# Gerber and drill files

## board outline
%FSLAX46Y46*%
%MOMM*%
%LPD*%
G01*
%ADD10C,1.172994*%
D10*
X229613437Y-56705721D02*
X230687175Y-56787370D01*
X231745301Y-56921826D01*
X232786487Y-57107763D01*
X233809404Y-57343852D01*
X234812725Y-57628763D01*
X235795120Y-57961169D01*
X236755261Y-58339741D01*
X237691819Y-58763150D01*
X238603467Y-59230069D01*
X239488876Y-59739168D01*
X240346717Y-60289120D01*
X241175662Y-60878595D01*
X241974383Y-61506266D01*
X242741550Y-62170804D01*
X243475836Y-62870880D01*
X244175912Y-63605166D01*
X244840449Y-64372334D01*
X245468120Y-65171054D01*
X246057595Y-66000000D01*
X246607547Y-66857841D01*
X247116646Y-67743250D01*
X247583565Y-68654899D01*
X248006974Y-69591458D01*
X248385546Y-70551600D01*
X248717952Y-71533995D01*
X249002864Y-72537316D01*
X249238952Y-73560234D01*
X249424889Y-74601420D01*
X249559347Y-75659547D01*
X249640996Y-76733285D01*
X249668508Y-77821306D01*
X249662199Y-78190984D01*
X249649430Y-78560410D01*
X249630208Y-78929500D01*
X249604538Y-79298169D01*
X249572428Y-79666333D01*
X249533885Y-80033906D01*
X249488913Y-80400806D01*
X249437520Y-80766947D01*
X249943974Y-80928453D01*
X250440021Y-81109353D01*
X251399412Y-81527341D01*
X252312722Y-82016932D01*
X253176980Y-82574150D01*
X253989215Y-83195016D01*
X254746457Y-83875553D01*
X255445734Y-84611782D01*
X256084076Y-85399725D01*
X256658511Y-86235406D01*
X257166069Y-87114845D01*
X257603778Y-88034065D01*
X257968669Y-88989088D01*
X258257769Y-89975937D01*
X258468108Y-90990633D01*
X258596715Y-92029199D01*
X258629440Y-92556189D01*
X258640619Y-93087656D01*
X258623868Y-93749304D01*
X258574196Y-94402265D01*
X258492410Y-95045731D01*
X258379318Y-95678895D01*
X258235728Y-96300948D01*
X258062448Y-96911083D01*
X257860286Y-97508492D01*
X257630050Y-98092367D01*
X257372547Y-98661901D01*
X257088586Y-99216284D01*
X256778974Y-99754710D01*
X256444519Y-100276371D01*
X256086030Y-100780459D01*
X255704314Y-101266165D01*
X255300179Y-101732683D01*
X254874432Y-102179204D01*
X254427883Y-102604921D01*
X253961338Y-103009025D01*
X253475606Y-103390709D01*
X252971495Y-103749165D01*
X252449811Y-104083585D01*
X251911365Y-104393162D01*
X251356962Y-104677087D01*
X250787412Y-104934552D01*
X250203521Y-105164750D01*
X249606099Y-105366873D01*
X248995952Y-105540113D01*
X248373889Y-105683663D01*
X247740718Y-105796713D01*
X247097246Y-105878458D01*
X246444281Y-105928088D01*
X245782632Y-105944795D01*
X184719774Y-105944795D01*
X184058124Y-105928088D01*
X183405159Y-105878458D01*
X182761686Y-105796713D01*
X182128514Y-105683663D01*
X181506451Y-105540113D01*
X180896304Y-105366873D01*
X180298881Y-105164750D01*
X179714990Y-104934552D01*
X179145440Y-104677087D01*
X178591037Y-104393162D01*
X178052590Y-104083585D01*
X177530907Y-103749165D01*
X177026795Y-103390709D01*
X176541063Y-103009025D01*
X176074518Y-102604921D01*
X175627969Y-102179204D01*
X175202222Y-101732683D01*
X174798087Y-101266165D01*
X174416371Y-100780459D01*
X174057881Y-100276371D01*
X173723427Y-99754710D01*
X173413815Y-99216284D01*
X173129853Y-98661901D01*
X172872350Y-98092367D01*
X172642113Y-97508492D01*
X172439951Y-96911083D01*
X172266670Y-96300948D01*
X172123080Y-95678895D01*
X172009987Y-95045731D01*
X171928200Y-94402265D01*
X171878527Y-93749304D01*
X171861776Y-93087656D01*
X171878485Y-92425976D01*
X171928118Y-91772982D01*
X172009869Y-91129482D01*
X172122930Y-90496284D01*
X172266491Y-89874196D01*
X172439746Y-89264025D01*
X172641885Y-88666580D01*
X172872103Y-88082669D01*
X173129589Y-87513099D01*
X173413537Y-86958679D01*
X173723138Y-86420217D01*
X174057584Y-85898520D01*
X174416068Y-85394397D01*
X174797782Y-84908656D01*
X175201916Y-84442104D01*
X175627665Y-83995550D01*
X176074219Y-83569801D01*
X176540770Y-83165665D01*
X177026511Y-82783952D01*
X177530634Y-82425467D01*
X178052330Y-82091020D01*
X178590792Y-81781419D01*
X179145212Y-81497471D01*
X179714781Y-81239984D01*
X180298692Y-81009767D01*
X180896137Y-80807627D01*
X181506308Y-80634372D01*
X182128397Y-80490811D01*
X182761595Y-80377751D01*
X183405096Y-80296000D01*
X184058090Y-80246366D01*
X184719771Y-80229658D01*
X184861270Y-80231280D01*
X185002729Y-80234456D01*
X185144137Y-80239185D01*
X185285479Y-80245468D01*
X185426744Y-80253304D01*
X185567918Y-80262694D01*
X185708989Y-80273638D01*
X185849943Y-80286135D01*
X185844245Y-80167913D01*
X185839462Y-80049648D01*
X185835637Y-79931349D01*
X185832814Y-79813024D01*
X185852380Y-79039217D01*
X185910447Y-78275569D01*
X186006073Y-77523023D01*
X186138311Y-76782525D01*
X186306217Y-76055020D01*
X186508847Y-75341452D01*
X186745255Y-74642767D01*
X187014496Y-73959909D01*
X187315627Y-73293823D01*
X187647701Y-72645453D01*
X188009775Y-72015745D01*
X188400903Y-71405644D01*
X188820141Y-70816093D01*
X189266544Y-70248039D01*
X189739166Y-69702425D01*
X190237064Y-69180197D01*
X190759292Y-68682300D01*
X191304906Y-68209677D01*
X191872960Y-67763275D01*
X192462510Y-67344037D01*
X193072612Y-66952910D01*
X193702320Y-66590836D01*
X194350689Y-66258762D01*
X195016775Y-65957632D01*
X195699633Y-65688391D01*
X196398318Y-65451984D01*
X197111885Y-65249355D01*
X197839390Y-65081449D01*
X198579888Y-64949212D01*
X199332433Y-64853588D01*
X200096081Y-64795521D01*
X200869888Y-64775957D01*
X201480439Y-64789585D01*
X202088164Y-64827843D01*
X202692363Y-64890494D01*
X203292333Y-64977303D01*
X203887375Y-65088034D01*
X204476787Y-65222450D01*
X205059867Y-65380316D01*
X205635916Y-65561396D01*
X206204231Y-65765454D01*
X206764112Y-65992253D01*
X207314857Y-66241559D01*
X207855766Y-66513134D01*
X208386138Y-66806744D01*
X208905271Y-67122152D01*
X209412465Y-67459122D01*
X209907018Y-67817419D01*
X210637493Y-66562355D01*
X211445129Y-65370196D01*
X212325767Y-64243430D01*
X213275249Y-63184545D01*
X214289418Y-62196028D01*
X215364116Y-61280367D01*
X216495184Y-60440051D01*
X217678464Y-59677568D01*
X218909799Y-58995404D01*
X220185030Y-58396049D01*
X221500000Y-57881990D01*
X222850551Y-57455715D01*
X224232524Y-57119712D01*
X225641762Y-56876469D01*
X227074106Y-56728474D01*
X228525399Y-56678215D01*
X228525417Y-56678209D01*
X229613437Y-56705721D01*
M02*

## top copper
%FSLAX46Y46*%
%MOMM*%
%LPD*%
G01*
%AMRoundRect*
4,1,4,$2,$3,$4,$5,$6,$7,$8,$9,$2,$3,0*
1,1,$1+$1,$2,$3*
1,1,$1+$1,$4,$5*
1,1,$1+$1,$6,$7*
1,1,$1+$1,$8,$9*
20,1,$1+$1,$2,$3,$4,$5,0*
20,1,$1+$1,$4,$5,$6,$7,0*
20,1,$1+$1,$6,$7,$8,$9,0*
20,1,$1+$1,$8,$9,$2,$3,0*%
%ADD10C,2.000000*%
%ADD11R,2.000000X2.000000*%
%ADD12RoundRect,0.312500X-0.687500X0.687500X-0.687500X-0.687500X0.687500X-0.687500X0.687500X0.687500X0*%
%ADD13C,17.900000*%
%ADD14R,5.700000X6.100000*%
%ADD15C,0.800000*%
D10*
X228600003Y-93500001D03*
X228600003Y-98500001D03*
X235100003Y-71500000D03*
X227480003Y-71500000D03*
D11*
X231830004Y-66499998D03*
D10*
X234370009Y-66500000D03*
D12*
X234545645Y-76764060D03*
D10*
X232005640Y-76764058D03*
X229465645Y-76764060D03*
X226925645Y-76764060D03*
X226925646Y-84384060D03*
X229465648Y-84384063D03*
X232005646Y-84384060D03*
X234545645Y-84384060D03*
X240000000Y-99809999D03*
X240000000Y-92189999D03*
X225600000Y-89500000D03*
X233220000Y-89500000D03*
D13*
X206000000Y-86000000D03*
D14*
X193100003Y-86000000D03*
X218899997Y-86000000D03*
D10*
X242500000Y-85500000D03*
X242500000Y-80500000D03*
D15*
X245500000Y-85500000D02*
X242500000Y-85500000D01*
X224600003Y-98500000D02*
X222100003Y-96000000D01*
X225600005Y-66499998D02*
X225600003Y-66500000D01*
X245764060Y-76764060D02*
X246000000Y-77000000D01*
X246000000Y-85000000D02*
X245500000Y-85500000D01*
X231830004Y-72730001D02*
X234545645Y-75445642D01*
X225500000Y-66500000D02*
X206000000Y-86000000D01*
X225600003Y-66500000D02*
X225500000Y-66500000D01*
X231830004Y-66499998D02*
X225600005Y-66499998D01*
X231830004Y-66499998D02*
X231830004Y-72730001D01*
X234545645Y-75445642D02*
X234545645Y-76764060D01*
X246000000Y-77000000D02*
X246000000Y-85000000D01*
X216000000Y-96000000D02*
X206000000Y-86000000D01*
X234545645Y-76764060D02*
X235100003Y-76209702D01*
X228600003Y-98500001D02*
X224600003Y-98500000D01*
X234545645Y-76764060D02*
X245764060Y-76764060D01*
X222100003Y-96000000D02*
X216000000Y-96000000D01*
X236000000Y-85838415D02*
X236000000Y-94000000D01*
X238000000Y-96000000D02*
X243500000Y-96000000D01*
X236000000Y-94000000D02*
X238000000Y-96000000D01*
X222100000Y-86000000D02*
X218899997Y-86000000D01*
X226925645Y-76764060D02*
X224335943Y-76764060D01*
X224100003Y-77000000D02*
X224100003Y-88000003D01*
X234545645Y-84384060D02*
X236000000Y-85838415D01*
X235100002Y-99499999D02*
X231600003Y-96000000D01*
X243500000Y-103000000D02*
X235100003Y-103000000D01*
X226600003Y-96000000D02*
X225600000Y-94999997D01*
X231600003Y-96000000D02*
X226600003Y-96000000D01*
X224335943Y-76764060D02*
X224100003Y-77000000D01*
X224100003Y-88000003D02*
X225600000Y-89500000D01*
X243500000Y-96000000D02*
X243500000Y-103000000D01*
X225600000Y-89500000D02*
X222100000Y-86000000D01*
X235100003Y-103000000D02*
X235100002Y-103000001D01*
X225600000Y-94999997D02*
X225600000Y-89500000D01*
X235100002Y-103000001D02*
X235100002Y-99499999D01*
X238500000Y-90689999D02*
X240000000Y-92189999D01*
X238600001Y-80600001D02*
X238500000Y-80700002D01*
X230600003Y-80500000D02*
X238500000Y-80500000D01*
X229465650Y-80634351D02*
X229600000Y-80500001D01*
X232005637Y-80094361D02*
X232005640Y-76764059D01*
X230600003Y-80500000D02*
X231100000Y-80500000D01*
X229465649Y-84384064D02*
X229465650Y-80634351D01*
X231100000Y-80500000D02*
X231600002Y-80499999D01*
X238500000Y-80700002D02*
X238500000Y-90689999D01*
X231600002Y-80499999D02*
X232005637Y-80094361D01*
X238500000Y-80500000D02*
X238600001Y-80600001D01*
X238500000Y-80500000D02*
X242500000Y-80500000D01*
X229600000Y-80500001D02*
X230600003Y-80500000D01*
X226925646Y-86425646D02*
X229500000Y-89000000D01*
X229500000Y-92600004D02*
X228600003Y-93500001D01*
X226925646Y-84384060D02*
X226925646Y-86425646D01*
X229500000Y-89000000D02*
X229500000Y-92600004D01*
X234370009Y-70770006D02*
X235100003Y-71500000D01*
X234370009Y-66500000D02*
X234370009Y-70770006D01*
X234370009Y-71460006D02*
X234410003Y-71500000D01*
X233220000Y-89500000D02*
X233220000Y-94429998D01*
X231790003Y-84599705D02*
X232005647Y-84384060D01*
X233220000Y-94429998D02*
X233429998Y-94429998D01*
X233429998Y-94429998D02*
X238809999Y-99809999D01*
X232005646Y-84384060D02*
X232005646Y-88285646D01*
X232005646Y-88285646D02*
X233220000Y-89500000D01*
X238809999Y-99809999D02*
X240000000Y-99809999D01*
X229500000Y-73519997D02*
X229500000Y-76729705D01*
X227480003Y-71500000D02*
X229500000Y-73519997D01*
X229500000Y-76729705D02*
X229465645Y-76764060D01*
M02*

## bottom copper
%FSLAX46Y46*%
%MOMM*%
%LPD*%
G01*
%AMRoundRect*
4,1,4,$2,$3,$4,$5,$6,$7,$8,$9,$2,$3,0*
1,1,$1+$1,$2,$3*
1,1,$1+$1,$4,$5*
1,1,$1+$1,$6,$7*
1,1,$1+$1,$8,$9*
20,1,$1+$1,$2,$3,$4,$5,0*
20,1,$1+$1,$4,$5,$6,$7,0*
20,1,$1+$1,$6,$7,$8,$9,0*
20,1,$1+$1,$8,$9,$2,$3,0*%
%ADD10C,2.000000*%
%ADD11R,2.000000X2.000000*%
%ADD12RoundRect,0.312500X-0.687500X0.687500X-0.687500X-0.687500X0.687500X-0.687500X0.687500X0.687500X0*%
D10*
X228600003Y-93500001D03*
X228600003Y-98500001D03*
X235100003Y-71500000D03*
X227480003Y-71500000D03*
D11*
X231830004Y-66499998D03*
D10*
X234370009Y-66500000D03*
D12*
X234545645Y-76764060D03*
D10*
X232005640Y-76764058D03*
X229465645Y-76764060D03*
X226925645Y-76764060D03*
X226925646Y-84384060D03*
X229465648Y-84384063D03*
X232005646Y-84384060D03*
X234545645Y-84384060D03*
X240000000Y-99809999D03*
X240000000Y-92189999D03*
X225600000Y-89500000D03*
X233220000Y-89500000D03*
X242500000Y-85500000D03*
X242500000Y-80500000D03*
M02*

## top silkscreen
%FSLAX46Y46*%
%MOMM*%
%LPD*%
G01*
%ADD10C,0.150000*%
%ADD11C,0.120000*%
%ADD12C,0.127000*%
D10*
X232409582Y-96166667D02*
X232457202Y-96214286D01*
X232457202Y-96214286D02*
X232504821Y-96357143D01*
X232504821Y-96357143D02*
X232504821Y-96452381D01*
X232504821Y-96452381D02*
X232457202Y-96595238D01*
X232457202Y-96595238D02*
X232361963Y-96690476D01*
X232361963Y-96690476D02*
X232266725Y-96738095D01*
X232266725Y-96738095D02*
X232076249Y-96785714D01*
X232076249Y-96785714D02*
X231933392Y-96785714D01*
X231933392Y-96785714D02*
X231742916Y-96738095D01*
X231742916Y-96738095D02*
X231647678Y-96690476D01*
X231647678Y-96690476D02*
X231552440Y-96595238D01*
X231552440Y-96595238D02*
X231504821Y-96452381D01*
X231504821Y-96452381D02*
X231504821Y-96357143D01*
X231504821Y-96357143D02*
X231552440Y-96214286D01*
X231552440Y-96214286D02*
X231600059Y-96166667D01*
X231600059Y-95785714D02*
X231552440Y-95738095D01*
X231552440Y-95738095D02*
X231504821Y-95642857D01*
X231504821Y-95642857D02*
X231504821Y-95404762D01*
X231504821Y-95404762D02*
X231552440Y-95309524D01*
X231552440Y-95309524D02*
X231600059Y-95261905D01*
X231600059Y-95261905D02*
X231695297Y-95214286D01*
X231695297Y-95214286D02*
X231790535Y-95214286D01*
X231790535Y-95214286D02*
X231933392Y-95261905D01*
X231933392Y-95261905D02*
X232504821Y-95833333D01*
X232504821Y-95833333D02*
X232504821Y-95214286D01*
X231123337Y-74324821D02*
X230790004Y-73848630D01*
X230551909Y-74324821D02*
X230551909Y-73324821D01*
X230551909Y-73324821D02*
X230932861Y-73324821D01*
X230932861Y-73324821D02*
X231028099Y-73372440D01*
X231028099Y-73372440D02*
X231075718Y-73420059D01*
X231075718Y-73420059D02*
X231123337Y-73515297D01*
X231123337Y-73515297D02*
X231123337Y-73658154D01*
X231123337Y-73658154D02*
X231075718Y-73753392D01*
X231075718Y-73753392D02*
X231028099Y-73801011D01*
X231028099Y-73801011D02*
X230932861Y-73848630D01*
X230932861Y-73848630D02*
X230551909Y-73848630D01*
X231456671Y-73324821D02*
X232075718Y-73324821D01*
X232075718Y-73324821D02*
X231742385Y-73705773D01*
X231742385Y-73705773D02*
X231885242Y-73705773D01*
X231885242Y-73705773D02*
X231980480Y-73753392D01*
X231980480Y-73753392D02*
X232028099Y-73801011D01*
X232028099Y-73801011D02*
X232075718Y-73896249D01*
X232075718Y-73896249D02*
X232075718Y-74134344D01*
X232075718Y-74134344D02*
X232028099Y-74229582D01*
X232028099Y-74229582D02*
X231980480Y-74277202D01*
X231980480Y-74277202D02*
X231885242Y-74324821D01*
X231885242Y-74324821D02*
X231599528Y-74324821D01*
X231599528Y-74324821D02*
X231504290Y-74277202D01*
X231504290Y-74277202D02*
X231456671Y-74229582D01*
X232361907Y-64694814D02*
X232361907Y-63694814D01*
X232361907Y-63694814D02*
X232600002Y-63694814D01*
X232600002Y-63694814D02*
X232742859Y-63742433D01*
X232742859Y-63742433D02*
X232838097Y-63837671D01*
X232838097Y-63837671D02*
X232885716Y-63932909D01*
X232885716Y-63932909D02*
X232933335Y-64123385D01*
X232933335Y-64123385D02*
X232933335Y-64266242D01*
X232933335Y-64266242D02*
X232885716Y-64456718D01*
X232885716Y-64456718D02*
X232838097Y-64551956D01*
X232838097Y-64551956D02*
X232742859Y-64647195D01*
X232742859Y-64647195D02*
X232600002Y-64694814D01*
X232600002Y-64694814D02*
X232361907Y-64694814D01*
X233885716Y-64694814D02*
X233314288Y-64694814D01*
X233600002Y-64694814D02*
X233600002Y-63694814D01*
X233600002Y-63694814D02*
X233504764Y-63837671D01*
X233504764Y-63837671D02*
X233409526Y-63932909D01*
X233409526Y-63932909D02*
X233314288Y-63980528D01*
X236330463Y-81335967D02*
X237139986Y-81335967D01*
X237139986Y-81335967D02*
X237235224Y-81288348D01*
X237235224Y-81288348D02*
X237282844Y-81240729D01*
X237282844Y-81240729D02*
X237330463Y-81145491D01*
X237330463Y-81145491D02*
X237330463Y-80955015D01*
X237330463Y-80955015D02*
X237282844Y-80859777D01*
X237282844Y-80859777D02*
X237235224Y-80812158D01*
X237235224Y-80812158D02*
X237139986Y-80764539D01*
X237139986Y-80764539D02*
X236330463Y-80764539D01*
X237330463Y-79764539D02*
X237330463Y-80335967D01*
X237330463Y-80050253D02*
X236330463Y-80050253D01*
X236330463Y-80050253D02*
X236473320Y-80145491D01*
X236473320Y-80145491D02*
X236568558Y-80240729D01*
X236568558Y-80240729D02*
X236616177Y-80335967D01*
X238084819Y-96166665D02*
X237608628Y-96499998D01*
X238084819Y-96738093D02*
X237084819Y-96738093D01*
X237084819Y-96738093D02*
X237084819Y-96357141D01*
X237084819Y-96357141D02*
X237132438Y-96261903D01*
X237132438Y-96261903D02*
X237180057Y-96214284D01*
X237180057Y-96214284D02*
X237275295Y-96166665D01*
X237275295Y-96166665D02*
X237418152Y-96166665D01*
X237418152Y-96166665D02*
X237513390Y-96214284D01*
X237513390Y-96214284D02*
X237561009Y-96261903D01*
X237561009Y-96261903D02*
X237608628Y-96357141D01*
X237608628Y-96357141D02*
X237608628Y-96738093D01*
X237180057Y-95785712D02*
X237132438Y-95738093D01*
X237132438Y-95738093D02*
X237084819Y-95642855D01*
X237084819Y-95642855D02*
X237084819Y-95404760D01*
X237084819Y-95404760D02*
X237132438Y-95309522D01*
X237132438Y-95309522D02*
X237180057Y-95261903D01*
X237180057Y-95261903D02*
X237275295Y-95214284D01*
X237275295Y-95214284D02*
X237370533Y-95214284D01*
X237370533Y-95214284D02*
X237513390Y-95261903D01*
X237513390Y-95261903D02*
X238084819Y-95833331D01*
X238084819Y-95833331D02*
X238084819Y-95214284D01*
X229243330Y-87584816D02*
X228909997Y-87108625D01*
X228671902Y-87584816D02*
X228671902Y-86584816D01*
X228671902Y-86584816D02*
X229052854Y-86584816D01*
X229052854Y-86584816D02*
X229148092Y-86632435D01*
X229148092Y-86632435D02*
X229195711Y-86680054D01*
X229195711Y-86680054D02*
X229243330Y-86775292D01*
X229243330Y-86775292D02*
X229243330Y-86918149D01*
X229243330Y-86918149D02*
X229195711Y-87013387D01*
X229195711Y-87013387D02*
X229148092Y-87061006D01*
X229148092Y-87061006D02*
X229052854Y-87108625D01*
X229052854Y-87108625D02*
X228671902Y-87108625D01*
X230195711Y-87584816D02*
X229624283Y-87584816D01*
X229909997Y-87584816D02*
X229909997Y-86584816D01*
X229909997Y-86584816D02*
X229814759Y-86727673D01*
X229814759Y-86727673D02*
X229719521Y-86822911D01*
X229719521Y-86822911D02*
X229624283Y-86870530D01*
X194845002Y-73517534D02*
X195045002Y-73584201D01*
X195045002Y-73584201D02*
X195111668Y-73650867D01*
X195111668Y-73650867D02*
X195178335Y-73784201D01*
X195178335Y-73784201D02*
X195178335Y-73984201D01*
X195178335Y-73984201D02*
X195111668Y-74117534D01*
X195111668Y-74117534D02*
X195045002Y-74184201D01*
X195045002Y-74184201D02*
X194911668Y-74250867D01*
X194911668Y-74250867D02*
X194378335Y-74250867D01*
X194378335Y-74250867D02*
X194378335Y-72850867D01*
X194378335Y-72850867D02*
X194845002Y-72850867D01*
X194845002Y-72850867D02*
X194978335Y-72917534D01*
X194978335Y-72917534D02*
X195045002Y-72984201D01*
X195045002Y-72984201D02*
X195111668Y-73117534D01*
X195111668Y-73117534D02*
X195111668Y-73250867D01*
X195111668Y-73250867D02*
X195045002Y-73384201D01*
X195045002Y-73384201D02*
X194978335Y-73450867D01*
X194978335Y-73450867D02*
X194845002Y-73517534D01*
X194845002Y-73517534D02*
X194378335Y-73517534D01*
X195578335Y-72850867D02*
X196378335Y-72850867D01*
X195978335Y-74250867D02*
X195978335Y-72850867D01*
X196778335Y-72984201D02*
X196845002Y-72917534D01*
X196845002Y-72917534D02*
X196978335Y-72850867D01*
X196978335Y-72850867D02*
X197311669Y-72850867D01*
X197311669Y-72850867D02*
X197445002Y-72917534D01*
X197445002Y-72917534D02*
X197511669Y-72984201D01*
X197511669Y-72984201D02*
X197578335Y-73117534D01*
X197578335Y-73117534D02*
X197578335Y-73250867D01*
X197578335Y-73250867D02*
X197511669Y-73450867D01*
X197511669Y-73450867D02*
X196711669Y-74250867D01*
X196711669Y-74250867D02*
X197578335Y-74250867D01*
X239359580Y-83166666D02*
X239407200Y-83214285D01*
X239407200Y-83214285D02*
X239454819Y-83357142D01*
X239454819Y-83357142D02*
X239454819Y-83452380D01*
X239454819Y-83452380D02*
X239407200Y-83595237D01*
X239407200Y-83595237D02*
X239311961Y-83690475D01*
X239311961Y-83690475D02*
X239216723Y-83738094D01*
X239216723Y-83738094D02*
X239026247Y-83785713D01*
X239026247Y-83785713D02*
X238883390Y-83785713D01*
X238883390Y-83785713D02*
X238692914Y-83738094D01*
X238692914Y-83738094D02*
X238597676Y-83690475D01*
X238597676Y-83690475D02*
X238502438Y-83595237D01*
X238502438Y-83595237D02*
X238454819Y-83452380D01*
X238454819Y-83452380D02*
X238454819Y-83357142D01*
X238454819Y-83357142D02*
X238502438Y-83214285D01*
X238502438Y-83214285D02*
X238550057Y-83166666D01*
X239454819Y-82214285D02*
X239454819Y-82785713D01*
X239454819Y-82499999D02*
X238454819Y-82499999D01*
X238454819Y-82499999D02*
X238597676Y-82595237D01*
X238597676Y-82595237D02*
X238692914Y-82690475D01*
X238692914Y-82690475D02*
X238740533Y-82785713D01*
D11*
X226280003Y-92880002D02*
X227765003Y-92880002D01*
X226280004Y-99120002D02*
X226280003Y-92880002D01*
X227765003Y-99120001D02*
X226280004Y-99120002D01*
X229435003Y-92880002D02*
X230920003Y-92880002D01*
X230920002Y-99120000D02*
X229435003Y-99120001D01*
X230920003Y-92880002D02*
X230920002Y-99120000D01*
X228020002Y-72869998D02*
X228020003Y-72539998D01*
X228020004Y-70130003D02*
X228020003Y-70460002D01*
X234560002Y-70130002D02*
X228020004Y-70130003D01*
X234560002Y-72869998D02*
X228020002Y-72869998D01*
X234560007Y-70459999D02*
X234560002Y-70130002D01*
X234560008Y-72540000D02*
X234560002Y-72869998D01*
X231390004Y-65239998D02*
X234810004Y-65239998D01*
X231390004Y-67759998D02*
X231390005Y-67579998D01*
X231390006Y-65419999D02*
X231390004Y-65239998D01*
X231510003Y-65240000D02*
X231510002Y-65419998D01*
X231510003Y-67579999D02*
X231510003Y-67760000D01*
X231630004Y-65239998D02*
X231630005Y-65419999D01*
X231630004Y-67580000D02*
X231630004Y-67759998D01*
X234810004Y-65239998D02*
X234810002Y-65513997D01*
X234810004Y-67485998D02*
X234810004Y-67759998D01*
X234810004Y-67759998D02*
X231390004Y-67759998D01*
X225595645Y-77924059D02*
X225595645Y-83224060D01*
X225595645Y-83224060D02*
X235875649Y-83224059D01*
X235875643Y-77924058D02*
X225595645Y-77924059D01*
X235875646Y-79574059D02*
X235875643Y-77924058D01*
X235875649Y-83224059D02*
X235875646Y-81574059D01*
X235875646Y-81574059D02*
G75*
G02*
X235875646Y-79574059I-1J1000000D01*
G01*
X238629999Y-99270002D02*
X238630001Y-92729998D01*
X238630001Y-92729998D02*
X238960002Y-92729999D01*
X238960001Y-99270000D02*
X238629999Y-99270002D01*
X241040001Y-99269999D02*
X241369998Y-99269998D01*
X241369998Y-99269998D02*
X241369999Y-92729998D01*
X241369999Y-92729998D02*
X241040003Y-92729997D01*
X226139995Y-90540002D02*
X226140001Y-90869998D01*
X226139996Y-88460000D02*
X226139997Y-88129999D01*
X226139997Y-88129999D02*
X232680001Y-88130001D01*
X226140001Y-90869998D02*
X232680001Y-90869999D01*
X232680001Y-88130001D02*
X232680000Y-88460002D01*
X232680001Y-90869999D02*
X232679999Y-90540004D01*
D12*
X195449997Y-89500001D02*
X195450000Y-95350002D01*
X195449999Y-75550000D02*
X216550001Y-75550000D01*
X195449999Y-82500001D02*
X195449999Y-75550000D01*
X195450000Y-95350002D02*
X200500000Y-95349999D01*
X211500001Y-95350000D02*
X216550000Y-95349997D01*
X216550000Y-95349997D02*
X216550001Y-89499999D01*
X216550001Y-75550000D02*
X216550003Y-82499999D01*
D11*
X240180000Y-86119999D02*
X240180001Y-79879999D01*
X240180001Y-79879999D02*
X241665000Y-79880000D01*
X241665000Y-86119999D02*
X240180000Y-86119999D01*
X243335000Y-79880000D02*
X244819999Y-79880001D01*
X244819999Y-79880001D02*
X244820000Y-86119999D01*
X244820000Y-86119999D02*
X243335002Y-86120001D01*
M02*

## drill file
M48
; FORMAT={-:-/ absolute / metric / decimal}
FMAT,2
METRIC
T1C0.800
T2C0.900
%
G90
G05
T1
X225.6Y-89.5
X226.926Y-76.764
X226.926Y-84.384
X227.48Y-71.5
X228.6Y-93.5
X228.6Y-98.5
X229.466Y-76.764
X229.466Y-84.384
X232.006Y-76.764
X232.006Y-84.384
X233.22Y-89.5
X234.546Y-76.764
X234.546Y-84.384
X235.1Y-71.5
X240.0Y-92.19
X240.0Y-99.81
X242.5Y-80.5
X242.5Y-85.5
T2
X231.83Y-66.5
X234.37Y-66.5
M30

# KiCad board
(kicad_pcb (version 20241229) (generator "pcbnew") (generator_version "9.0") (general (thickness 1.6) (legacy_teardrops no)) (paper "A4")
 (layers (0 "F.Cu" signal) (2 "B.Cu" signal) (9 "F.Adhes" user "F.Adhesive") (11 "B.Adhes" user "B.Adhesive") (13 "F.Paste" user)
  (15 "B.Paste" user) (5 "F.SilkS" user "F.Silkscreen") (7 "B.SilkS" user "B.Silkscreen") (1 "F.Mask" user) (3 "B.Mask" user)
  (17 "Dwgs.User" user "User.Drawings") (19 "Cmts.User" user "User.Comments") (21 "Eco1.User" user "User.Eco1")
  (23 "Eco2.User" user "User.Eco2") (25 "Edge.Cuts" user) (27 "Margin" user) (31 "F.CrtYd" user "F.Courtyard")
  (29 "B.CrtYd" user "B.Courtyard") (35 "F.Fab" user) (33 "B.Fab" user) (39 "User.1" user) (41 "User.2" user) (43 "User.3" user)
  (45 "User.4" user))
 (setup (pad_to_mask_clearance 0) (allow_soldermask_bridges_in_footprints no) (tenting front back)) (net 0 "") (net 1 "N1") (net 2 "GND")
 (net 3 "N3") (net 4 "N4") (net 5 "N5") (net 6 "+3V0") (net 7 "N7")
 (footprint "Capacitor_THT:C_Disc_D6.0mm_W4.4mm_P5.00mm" (layer "F.Cu") (at 228.600003 93.500001 -90)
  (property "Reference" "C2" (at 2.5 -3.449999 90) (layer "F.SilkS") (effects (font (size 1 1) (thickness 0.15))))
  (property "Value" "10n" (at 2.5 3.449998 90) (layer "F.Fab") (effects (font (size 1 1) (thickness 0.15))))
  (fp_line (start -0.619999 2.32) (end -0.619999 0.835) (stroke (width 0.12) (type solid)) (layer "F.SilkS"))
  (fp_line (start 5.620001 2.319999) (end -0.619999 2.32) (stroke (width 0.12) (type solid)) (layer "F.SilkS"))
  (fp_line (start 5.62 0.835) (end 5.620001 2.319999) (stroke (width 0.12) (type solid)) (layer "F.SilkS"))
  (fp_line (start -0.619999 -0.835) (end -0.619999 -2.32) (stroke (width 0.12) (type solid)) (layer "F.SilkS"))
  (fp_line (start 5.619999 -2.319999) (end 5.62 -0.835) (stroke (width 0.12) (type solid)) (layer "F.SilkS"))
  (fp_line (start -0.619999 -2.32) (end 5.619999 -2.319999) (stroke (width 0.12) (type solid)) (layer "F.SilkS"))
  (pad "1" thru_hole circle (at 0 0 270) (size 2 2) (drill 0.8) (layers "*.Cu" "*.Mask") (remove_unused_layers no) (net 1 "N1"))
  (pad "2" thru_hole circle (at 5 0 270) (size 2 2) (drill 0.8) (layers "*.Cu" "*.Mask") (remove_unused_layers no) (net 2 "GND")))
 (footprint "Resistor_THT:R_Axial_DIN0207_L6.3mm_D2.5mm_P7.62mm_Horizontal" (layer "F.Cu") (at 235.100003 71.5 180)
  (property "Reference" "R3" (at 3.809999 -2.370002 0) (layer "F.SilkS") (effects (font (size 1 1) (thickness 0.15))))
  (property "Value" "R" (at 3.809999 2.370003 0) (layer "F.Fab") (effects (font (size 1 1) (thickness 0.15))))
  (fp_line (start 7.080001 -1.369998) (end 7.08 -1.039998) (stroke (width 0.12) (type solid)) (layer "F.SilkS"))
  (fp_line (start 7.079999 1.369997) (end 7.08 1.039998) (stroke (width 0.12) (type solid)) (layer "F.SilkS"))
  (fp_line (start 0.540001 1.369998) (end 7.079999 1.369997) (stroke (width 0.12) (type solid)) (layer "F.SilkS"))
  (fp_line (start 0.540001 -1.369998) (end 7.080001 -1.369998) (stroke (width 0.12) (type solid)) (layer "F.SilkS"))
  (fp_line (start 0.539996 1.040001) (end 0.540001 1.369998) (stroke (width 0.12) (type solid)) (layer "F.SilkS"))
  (fp_line (start 0.539995 -1.04) (end 0.540001 -1.369998) (stroke (width 0.12) (type solid)) (layer "F.SilkS"))
  (pad "1" thru_hole circle (at 0 0 180) (size 2 2) (drill 0.8) (layers "*.Cu" "*.Mask") (remove_unused_layers no) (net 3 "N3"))
  (pad "2" thru_hole circle (at 7.62 0 180) (size 2 2) (drill 0.8) (layers "*.Cu" "*.Mask") (remove_unused_layers no) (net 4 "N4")))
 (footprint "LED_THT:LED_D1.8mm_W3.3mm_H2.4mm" (layer "F.Cu") (at 231.830004 66.499998)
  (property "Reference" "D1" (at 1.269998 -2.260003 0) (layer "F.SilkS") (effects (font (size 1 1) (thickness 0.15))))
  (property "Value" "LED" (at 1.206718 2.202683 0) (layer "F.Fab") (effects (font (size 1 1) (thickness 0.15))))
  (fp_line (start -0.44 -1.26) (end 2.98 -1.26) (stroke (width 0.12) (type solid)) (layer "F.SilkS"))
  (fp_line (start -0.44 1.26) (end -0.439999 1.08) (stroke (width 0.12) (type solid)) (layer "F.SilkS"))
  (fp_line (start -0.439998 -1.079999) (end -0.44 -1.26) (stroke (width 0.12) (type solid)) (layer "F.SilkS"))
  (fp_line (start -0.320001 -1.259998) (end -0.320002 -1.08) (stroke (width 0.12) (type solid)) (layer "F.SilkS"))
  (fp_line (start -0.320001 1.080001) (end -0.320001 1.260002) (stroke (width 0.12) (type solid)) (layer "F.SilkS"))
  (fp_line (start -0.2 -1.26) (end -0.199999 -1.079999) (stroke (width 0.12) (type solid)) (layer "F.SilkS"))
  (fp_line (start -0.2 1.080002) (end -0.2 1.26) (stroke (width 0.12) (type solid)) (layer "F.SilkS"))
  (fp_line (start 2.98 -1.26) (end 2.979998 -0.986001) (stroke (width 0.12) (type solid)) (layer "F.SilkS"))
  (fp_line (start 2.98 0.986) (end 2.98 1.26) (stroke (width 0.12) (type solid)) (layer "F.SilkS"))
  (fp_line (start 2.98 1.26) (end -0.44 1.26) (stroke (width 0.12) (type solid)) (layer "F.SilkS"))
  (pad "1" thru_hole rect (at 0 0) (size 2 2) (drill 0.9) (layers "*.Cu" "*.Mask") (remove_unused_layers no) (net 2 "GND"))
  (pad "2" thru_hole circle (at 2.540005 0.000002) (size 2 2) (drill 0.9) (layers "*.Cu" "*.Mask") (remove_unused_layers no) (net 3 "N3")))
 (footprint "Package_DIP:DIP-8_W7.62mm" (layer "F.Cu") (at 234.545645 76.76406 -90)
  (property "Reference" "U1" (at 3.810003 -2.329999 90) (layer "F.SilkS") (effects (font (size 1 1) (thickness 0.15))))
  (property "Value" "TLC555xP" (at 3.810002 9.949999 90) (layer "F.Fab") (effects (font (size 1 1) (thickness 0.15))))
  (fp_line (start 1.159999 8.95) (end 6.46 8.95) (stroke (width 0.12) (type solid)) (layer "F.SilkS"))
  (fp_line (start 6.46 8.95) (end 6.459999 -1.330004) (stroke (width 0.12) (type solid)) (layer "F.SilkS"))
  (fp_line (start 1.159998 -1.329998) (end 1.159999 8.95) (stroke (width 0.12) (type solid)) (layer "F.SilkS"))
  (fp_line (start 2.809999 -1.330001) (end 1.159998 -1.329998) (stroke (width 0.12) (type solid)) (layer "F.SilkS"))
  (fp_line (start 6.459999 -1.330004) (end 4.809999 -1.330001) (stroke (width 0.12) (type solid)) (layer "F.SilkS"))
  (fp_arc (start 4.809999 -1.330001) (mid 3.81 -0.33) (end 2.809999 -1.330001) (stroke (width 0.12) (type solid)) (layer "F.SilkS"))
  (pad "1" thru_hole roundrect (at 0 0 270) (size 2 2) (drill 0.8) (layers "*.Cu" "*.Mask") (remove_unused_layers no)
   (roundrect_rratio 0.15625) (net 2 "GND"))
  (pad "2" thru_hole circle (at -0.000002 2.540005 270) (size 2 2) (drill 0.8) (layers "*.Cu" "*.Mask") (remove_unused_layers no)
   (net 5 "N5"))
  (pad "3" thru_hole circle (at 0 5.08 270) (size 2 2) (drill 0.8) (layers "*.Cu" "*.Mask") (remove_unused_layers no) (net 4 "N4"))
  (pad "4" thru_hole circle (at 0 7.62 270) (size 2 2) (drill 0.8) (layers "*.Cu" "*.Mask") (remove_unused_layers no) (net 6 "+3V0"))
  (pad "5" thru_hole circle (at 7.62 7.619999 270) (size 2 2) (drill 0.8) (layers "*.Cu" "*.Mask") (remove_unused_layers no) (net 1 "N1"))
  (pad "6" thru_hole circle (at 7.620003 5.079997 270) (size 2 2) (drill 0.8) (layers "*.Cu" "*.Mask") (remove_unused_layers no)
   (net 5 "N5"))
  (pad "7" thru_hole circle (at 7.62 2.539999 270) (size 2 2) (drill 0.8) (layers "*.Cu" "*.Mask") (remove_unused_layers no) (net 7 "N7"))
  (pad "8" thru_hole circle (at 7.62 0 270) (size 2 2) (drill 0.8) (layers "*.Cu" "*.Mask") (remove_unused_layers no) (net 6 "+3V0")))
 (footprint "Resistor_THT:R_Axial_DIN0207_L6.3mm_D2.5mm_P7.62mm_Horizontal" (layer "F.Cu") (at 240 99.809999 90)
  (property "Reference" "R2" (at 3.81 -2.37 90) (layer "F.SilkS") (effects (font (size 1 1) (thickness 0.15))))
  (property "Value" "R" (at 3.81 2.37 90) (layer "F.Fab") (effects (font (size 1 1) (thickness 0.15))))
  (fp_line (start 0.539997 -1.370001) (end 7.080001 -1.369999) (stroke (width 0.12) (type solid)) (layer "F.SilkS"))
  (fp_line (start 7.080001 -1.369999) (end 7.08 -1.039998) (stroke (width 0.12) (type solid)) (layer "F.SilkS"))
  (fp_line (start 0.539999 -1.039999) (end 0.539997 -1.370001) (stroke (width 0.12) (type solid)) (layer "F.SilkS"))
  (fp_line (start 0.54 1.040001) (end 0.540001 1.369998) (stroke (width 0.12) (type solid)) (layer "F.SilkS"))
  (fp_line (start 0.540001 1.369998) (end 7.080001 1.369999) (stroke (width 0.12) (type solid)) (layer "F.SilkS"))
  (fp_line (start 7.080001 1.369999) (end 7.080002 1.040003) (stroke (width 0.12) (type solid)) (layer "F.SilkS"))
  (pad "1" thru_hole circle (at 0 0 90) (size 2 2) (drill 0.8) (layers "*.Cu" "*.Mask") (remove_unused_layers no) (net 7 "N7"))
  (pad "2" thru_hole circle (at 7.62 0 90) (size 2 2) (drill 0.8) (layers "*.Cu" "*.Mask") (remove_unused_layers no) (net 5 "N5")))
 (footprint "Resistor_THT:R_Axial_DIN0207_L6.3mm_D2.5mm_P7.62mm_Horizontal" (layer "F.Cu") (at 225.6 89.5)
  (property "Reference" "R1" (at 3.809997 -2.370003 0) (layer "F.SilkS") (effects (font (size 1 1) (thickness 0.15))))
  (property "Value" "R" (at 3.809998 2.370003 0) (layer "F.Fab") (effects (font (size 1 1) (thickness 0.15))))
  (fp_line (start 0.539995 1.040002) (end 0.540001 1.369998) (stroke (width 0.12) (type solid)) (layer "F.SilkS"))
  (fp_line (start 0.539996 -1.04) (end 0.539997 -1.370001) (stroke (width 0.12) (type solid)) (layer "F.SilkS"))
  (fp_line (start 0.539997 -1.370001) (end 7.080001 -1.369999) (stroke (width 0.12) (type solid)) (layer "F.SilkS"))
  (fp_line (start 0.540001 1.369998) (end 7.080001 1.369999) (stroke (width 0.12) (type solid)) (layer "F.SilkS"))
  (fp_line (start 7.080001 -1.369999) (end 7.08 -1.039998) (stroke (width 0.12) (type solid)) (layer "F.SilkS"))
  (fp_line (start 7.080001 1.369999) (end 7.079999 1.040004) (stroke (width 0.12) (type solid)) (layer "F.SilkS"))
  (pad "1" thru_hole circle (at 0 0) (size 2 2) (drill 0.8) (layers "*.Cu" "*.Mask") (remove_unused_layers no) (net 6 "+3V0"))
  (pad "2" thru_hole circle (at 7.62 0) (size 2 2) (drill 0.8) (layers "*.Cu" "*.Mask") (remove_unused_layers no) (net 7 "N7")))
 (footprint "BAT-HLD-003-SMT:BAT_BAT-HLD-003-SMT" (layer "F.Cu") (at 206 86)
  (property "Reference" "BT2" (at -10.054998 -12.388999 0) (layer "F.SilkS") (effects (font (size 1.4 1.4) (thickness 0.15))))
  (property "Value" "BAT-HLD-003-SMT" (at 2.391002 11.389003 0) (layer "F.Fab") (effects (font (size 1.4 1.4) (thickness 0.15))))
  (fp_line (start -10.550003 3.500001) (end -10.55 9.350002) (stroke (width 0.127) (type solid)) (layer "F.SilkS"))
  (fp_line (start -10.550001 -10.45) (end 10.550001 -10.45) (stroke (width 0.127) (type solid)) (layer "F.SilkS"))
  (fp_line (start -10.550001 -3.499999) (end -10.550001 -10.45) (stroke (width 0.127) (type solid)) (layer "F.SilkS"))
  (fp_line (start -10.55 9.350002) (end -5.5 9.349999) (stroke (width 0.127) (type solid)) (layer "F.SilkS"))
  (fp_line (start 5.500001 9.35) (end 10.55 9.349997) (stroke (width 0.127) (type solid)) (layer "F.SilkS"))
  (fp_line (start 10.55 9.349997) (end 10.550001 3.499999) (stroke (width 0.127) (type solid)) (layer "F.SilkS"))
  (fp_line (start 10.550001 -10.45) (end 10.550003 -3.500001) (stroke (width 0.127) (type solid)) (layer "F.SilkS"))
  (pad "N" smd circle (at 0 0) (size 17.9 17.9) (layers "F.Cu" "F.Mask") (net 2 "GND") (solder_mask_margin 0.102))
  (pad "P1" smd rect (at -12.899997 0) (size 5.7 6.1) (layers "F.Cu" "F.Mask" "F.Paste") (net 6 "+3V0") (solder_mask_margin 0.102))
  (pad "P2" smd rect (at 12.899997 0) (size 5.7 6.1) (layers "F.Cu" "F.Mask" "F.Paste") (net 6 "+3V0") (solder_mask_margin 0.102)))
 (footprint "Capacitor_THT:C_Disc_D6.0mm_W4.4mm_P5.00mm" (layer "F.Cu") (at 242.5 85.5 90)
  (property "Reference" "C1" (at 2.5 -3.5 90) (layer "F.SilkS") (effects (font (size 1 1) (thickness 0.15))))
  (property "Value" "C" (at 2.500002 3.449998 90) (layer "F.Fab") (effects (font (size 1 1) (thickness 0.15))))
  (fp_line (start -0.619999 -2.32) (end 5.620001 -2.319999) (stroke (width 0.12) (type solid)) (layer "F.SilkS"))
  (fp_line (start 5.620001 -2.319999) (end 5.62 -0.835) (stroke (width 0.12) (type solid)) (layer "F.SilkS"))
  (fp_line (start -0.619999 -0.835) (end -0.619999 -2.32) (stroke (width 0.12) (type solid)) (layer "F.SilkS"))
  (fp_line (start 5.62 0.835) (end 5.619999 2.319999) (stroke (width 0.12) (type solid)) (layer "F.SilkS"))
  (fp_line (start 5.619999 2.319999) (end -0.619999 2.32) (stroke (width 0.12) (type solid)) (layer "F.SilkS"))
  (fp_line (start -0.619999 2.32) (end -0.620001 0.835002) (stroke (width 0.12) (type solid)) (layer "F.SilkS"))
  (pad "1" thru_hole circle (at 0 0 90) (size 2 2) (drill 0.8) (layers "*.Cu" "*.Mask") (remove_unused_layers no) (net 2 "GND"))
  (pad "2" thru_hole circle (at 5 0 90) (size 2 2) (drill 0.8) (layers "*.Cu" "*.Mask") (remove_unused_layers no) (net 5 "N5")))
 (gr_poly
  (pts (xy 229.613437 56.705721) (xy 230.687175 56.78737) (xy 231.745301 56.921826) (xy 232.786487 57.107763) (xy 233.809404 57.343852)
   (xy 234.812725 57.628763) (xy 235.79512 57.961169) (xy 236.755261 58.339741) (xy 237.691819 58.76315) (xy 238.603467 59.230069)
   (xy 239.488876 59.739168) (xy 240.346717 60.28912) (xy 241.175662 60.878595) (xy 241.974383 61.506266) (xy 242.74155 62.170804)
   (xy 243.475836 62.87088) (xy 244.175912 63.605166) (xy 244.840449 64.372334) (xy 245.46812 65.171054) (xy 246.057595 66)
   (xy 246.607547 66.857841) (xy 247.116646 67.74325) (xy 247.583565 68.654899) (xy 248.006974 69.591458) (xy 248.385546 70.5516)
   (xy 248.717952 71.533995) (xy 249.002864 72.537316) (xy 249.238952 73.560234) (xy 249.424889 74.60142) (xy 249.559347 75.659547)
   (xy 249.640996 76.733285) (xy 249.668508 77.821306) (xy 249.662199 78.190984) (xy 249.64943 78.56041) (xy 249.630208 78.9295)
   (xy 249.604538 79.298169) (xy 249.572428 79.666333) (xy 249.533885 80.033906) (xy 249.488913 80.400806) (xy 249.43752 80.766947)
   (xy 249.943974 80.928453) (xy 250.440021 81.109353) (xy 251.399412 81.527341) (xy 252.312722 82.016932) (xy 253.17698 82.57415)
   (xy 253.989215 83.195016) (xy 254.746457 83.875553) (xy 255.445734 84.611782) (xy 256.084076 85.399725) (xy 256.658511 86.235406)
   (xy 257.166069 87.114845) (xy 257.603778 88.034065) (xy 257.968669 88.989088) (xy 258.257769 89.975937) (xy 258.468108 90.990633)
   (xy 258.596715 92.029199) (xy 258.62944 92.556189) (xy 258.640619 93.087656) (xy 258.623868 93.749304) (xy 258.574196 94.402265)
   (xy 258.49241 95.045731) (xy 258.379318 95.678895) (xy 258.235728 96.300948) (xy 258.062448 96.911083) (xy 257.860286 97.508492)
   (xy 257.63005 98.092367) (xy 257.372547 98.661901) (xy 257.088586 99.216284) (xy 256.778974 99.75471) (xy 256.444519 100.276371)
   (xy 256.08603 100.780459) (xy 255.704314 101.266165) (xy 255.300179 101.732683) (xy 254.874432 102.179204) (xy 254.427883 102.604921)
   (xy 253.961338 103.009025) (xy 253.475606 103.390709) (xy 252.971495 103.749165) (xy 252.449811 104.083585) (xy 251.911365 104.393162)
   (xy 251.356962 104.677087) (xy 250.787412 104.934552) (xy 250.203521 105.16475) (xy 249.606099 105.366873) (xy 248.995952 105.540113)
   (xy 248.373889 105.683663) (xy 247.740718 105.796713) (xy 247.097246 105.878458) (xy 246.444281 105.928088) (xy 245.782632 105.944795)
   (xy 184.719774 105.944795) (xy 184.058124 105.928088) (xy 183.405159 105.878458) (xy 182.761686 105.796713) (xy 182.128514 105.683663)
   (xy 181.506451 105.540113) (xy 180.896304 105.366873) (xy 180.298881 105.16475) (xy 179.71499 104.934552) (xy 179.14544 104.677087)
   (xy 178.591037 104.393162) (xy 178.05259 104.083585) (xy 177.530907 103.749165) (xy 177.026795 103.390709) (xy 176.541063 103.009025)
   (xy 176.074518 102.604921) (xy 175.627969 102.179204) (xy 175.202222 101.732683) (xy 174.798087 101.266165) (xy 174.416371 100.780459)
   (xy 174.057881 100.276371) (xy 173.723427 99.75471) (xy 173.413815 99.216284) (xy 173.129853 98.661901) (xy 172.87235 98.092367)
   (xy 172.642113 97.508492) (xy 172.439951 96.911083) (xy 172.26667 96.300948) (xy 172.12308 95.678895) (xy 172.009987 95.045731)
   (xy 171.9282 94.402265) (xy 171.878527 93.749304) (xy 171.861776 93.087656) (xy 171.878485 92.425976) (xy 171.928118 91.772982)
   (xy 172.009869 91.129482) (xy 172.12293 90.496284) (xy 172.266491 89.874196) (xy 172.439746 89.264025) (xy 172.641885 88.66658)
   (xy 172.872103 88.082669) (xy 173.129589 87.513099) (xy 173.413537 86.958679) (xy 173.723138 86.420217) (xy 174.057584 85.89852)
   (xy 174.416068 85.394397) (xy 174.797782 84.908656) (xy 175.201916 84.442104) (xy 175.627665 83.99555) (xy 176.074219 83.569801)
   (xy 176.54077 83.165665) (xy 177.026511 82.783952) (xy 177.530634 82.425467) (xy 178.05233 82.09102) (xy 178.590792 81.781419)
   (xy 179.145212 81.497471) (xy 179.714781 81.239984) (xy 180.298692 81.009767) (xy 180.896137 80.807627) (xy 181.506308 80.634372)
   (xy 182.128397 80.490811) (xy 182.761595 80.377751) (xy 183.405096 80.296) (xy 184.05809 80.246366) (xy 184.719771 80.229658)
   (xy 184.86127 80.23128) (xy 185.002729 80.234456) (xy 185.144137 80.239185) (xy 185.285479 80.245468) (xy 185.426744 80.253304)
   (xy 185.567918 80.262694) (xy 185.708989 80.273638) (xy 185.849943 80.286135) (xy 185.844245 80.167913) (xy 185.839462 80.049648)
   (xy 185.835637 79.931349) (xy 185.832814 79.813024) (xy 185.85238 79.039217) (xy 185.910447 78.275569) (xy 186.006073 77.523023)
   (xy 186.138311 76.782525) (xy 186.306217 76.05502) (xy 186.508847 75.341452) (xy 186.745255 74.642767) (xy 187.014496 73.959909)
   (xy 187.315627 73.293823) (xy 187.647701 72.645453) (xy 188.009775 72.015745) (xy 188.400903 71.405644) (xy 188.820141 70.816093)
   (xy 189.266544 70.248039) (xy 189.739166 69.702425) (xy 190.237064 69.180197) (xy 190.759292 68.6823) (xy 191.304906 68.209677)
   (xy 191.87296 67.763275) (xy 192.46251 67.344037) (xy 193.072612 66.95291) (xy 193.70232 66.590836) (xy 194.350689 66.258762)
   (xy 195.016775 65.957632) (xy 195.699633 65.688391) (xy 196.398318 65.451984) (xy 197.111885 65.249355) (xy 197.83939 65.081449)
   (xy 198.579888 64.949212) (xy 199.332433 64.853588) (xy 200.096081 64.795521) (xy 200.869888 64.775957) (xy 201.480439 64.789585)
   (xy 202.088164 64.827843) (xy 202.692363 64.890494) (xy 203.292333 64.977303) (xy 203.887375 65.088034) (xy 204.476787 65.22245)
   (xy 205.059867 65.380316) (xy 205.635916 65.561396) (xy 206.204231 65.765454) (xy 206.764112 65.992253) (xy 207.314857 66.241559)
   (xy 207.855766 66.513134) (xy 208.386138 66.806744) (xy 208.905271 67.122152) (xy 209.412465 67.459122) (xy 209.907018 67.817419)
   (xy 210.637493 66.562355) (xy 211.445129 65.370196) (xy 212.325767 64.24343) (xy 213.275249 63.184545) (xy 214.289418 62.196028)
   (xy 215.364116 61.280367) (xy 216.495184 60.440051) (xy 217.678464 59.677568) (xy 218.909799 58.995404) (xy 220.18503 58.396049)
   (xy 221.5 57.88199) (xy 222.850551 57.455715) (xy 224.232524 57.119712) (xy 225.641762 56.876469) (xy 227.074106 56.728474)
   (xy 228.525399 56.678215) (xy 228.525417 56.678209))
  (stroke (width 1.172994) (type solid) (color 51 51 51 1)) (fill no) (layer "Edge.Cuts"))
 (segment (start 245.5 85.5) (end 242.5 85.5) (width 0.8) (layer "F.Cu") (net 2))
 (segment (start 224.600003 98.5) (end 222.100003 96) (width 0.8) (layer "F.Cu") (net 2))
 (segment (start 225.600005 66.499998) (end 225.600003 66.5) (width 0.8) (layer "F.Cu") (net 2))
 (segment (start 245.76406 76.76406) (end 246 77) (width 0.8) (layer "F.Cu") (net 2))
 (segment (start 246 85) (end 245.5 85.5) (width 0.8) (layer "F.Cu") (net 2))
 (segment (start 231.830004 72.730001) (end 234.545645 75.445642) (width 0.8) (layer "F.Cu") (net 2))
 (segment (start 225.5 66.5) (end 206 86) (width 0.8) (layer "F.Cu") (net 2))
 (segment (start 225.600003 66.5) (end 225.5 66.5) (width 0.8) (layer "F.Cu") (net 2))
 (segment (start 231.830004 66.499998) (end 225.600005 66.499998) (width 0.8) (layer "F.Cu") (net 2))
 (segment (start 231.830004 66.499998) (end 231.830004 72.730001) (width 0.8) (layer "F.Cu") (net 2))
 (segment (start 234.545645 75.445642) (end 234.545645 76.76406) (width 0.8) (layer "F.Cu") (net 2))
 (segment (start 246 77) (end 246 85) (width 0.8) (layer "F.Cu") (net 2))
 (segment (start 216 96) (end 206 86) (width 0.8) (layer "F.Cu") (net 2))
 (segment (start 234.545645 76.76406) (end 235.100003 76.209702) (width 0.8) (layer "F.Cu") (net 2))
 (segment (start 228.600003 98.500001) (end 224.600003 98.5) (width 0.8) (layer "F.Cu") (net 2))
 (segment (start 234.545645 76.76406) (end 245.76406 76.76406) (width 0.8) (layer "F.Cu") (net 2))
 (segment (start 222.100003 96) (end 216 96) (width 0.8) (layer "F.Cu") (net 2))
 (segment (start 236 85.838415) (end 236 94) (width 0.8) (layer "F.Cu") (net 6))
 (segment (start 238 96) (end 243.5 96) (width 0.8) (layer "F.Cu") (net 6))
 (segment (start 236 94) (end 238 96) (width 0.8) (layer "F.Cu") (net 6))
 (segment (start 222.1 86) (end 218.899997 86) (width 0.8) (layer "F.Cu") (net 6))
 (segment (start 226.925645 76.76406) (end 224.335943 76.76406) (width 0.8) (layer "F.Cu") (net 6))
 (segment (start 224.100003 77) (end 224.100003 88.000003) (width 0.8) (layer "F.Cu") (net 6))
 (segment (start 234.545645 84.38406) (end 236 85.838415) (width 0.8) (layer "F.Cu") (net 6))
 (segment (start 235.100002 99.499999) (end 231.600003 96) (width 0.8) (layer "F.Cu") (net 6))
 (segment (start 243.5 103) (end 235.100003 103) (width 0.8) (layer "F.Cu") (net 6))
 (segment (start 226.600003 96) (end 225.6 94.999997) (width 0.8) (layer "F.Cu") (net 6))
 (segment (start 231.600003 96) (end 226.600003 96) (width 0.8) (layer "F.Cu") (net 6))
 (segment (start 224.335943 76.76406) (end 224.100003 77) (width 0.8) (layer "F.Cu") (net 6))
 (segment (start 224.100003 88.000003) (end 225.6 89.5) (width 0.8) (layer "F.Cu") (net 6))
 (segment (start 243.5 96) (end 243.5 103) (width 0.8) (layer "F.Cu") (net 6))
 (segment (start 225.6 89.5) (end 222.1 86) (width 0.8) (layer "F.Cu") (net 6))
 (segment (start 235.100003 103) (end 235.100002 103.000001) (width 0.8) (layer "F.Cu") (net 6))
 (segment (start 225.6 94.999997) (end 225.6 89.5) (width 0.8) (layer "F.Cu") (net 6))
 (segment (start 235.100002 103.000001) (end 235.100002 99.499999) (width 0.8) (layer "F.Cu") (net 6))
 (segment (start 238.5 90.689999) (end 240 92.189999) (width 0.8) (layer "F.Cu") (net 5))
 (segment (start 238.600001 80.600001) (end 238.5 80.700002) (width 0.8) (layer "F.Cu") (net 5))
 (segment (start 230.600003 80.5) (end 238.5 80.5) (width 0.8) (layer "F.Cu") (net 5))
 (segment (start 229.46565 80.634351) (end 229.6 80.500001) (width 0.8) (layer "F.Cu") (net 5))
 (segment (start 232.005637 80.094361) (end 232.00564 76.764059) (width 0.8) (layer "F.Cu") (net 5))
 (segment (start 230.600003 80.5) (end 231.1 80.5) (width 0.8) (layer "F.Cu") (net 5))
 (segment (start 229.465649 84.384064) (end 229.46565 80.634351) (width 0.8) (layer "F.Cu") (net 5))
 (segment (start 231.1 80.5) (end 231.600002 80.499999) (width 0.8) (layer "F.Cu") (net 5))
 (segment (start 238.5 80.700002) (end 238.5 90.689999) (width 0.8) (layer "F.Cu") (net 5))
 (segment (start 231.600002 80.499999) (end 232.005637 80.094361) (width 0.8) (layer "F.Cu") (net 5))
 (segment (start 238.5 80.5) (end 238.600001 80.600001) (width 0.8) (layer "F.Cu") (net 5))
 (segment (start 238.5 80.5) (end 242.5 80.5) (width 0.8) (layer "F.Cu") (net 5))
 (segment (start 229.6 80.500001) (end 230.600003 80.5) (width 0.8) (layer "F.Cu") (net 5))
 (segment (start 226.925646 86.425646) (end 229.5 89) (width 0.8) (layer "F.Cu") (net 1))
 (segment (start 229.5 92.600004) (end 228.600003 93.500001) (width 0.8) (layer "F.Cu") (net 1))
 (segment (start 226.925646 84.38406) (end 226.925646 86.425646) (width 0.8) (layer "F.Cu") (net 1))
 (segment (start 229.5 89) (end 229.5 92.600004) (width 0.8) (layer "F.Cu") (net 1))
 (segment (start 234.370009 70.770006) (end 235.100003 71.5) (width 0.8) (layer "F.Cu") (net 3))
 (segment (start 234.370009 66.5) (end 234.370009 70.770006) (width 0.8) (layer "F.Cu") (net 3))
 (segment (start 234.370009 71.460006) (end 234.410003 71.5) (width 0.8) (layer "F.Cu") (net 3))
 (segment (start 233.22 89.5) (end 233.22 94.429998) (width 0.8) (layer "F.Cu") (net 7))
 (segment (start 231.790003 84.599705) (end 232.005647 84.38406) (width 0.8) (layer "F.Cu") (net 7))
 (segment (start 233.22 94.429998) (end 233.429998 94.429998) (width 0.8) (layer "F.Cu") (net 7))
 (segment (start 233.429998 94.429998) (end 238.809999 99.809999) (width 0.8) (layer "F.Cu") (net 7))
 (segment (start 232.005646 84.38406) (end 232.005646 88.285646) (width 0.8) (layer "F.Cu") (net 7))
 (segment (start 232.005646 88.285646) (end 233.22 89.5) (width 0.8) (layer "F.Cu") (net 7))
 (segment (start 238.809999 99.809999) (end 240 99.809999) (width 0.8) (layer "F.Cu") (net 7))
 (segment (start 229.5 73.519997) (end 229.5 76.729705) (width 0.8) (layer "F.Cu") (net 4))
 (segment (start 227.480003 71.5) (end 229.5 73.519997) (width 0.8) (layer "F.Cu") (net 4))
 (segment (start 229.5 76.729705) (end 229.465645 76.76406) (width 0.8) (layer "F.Cu") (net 4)))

